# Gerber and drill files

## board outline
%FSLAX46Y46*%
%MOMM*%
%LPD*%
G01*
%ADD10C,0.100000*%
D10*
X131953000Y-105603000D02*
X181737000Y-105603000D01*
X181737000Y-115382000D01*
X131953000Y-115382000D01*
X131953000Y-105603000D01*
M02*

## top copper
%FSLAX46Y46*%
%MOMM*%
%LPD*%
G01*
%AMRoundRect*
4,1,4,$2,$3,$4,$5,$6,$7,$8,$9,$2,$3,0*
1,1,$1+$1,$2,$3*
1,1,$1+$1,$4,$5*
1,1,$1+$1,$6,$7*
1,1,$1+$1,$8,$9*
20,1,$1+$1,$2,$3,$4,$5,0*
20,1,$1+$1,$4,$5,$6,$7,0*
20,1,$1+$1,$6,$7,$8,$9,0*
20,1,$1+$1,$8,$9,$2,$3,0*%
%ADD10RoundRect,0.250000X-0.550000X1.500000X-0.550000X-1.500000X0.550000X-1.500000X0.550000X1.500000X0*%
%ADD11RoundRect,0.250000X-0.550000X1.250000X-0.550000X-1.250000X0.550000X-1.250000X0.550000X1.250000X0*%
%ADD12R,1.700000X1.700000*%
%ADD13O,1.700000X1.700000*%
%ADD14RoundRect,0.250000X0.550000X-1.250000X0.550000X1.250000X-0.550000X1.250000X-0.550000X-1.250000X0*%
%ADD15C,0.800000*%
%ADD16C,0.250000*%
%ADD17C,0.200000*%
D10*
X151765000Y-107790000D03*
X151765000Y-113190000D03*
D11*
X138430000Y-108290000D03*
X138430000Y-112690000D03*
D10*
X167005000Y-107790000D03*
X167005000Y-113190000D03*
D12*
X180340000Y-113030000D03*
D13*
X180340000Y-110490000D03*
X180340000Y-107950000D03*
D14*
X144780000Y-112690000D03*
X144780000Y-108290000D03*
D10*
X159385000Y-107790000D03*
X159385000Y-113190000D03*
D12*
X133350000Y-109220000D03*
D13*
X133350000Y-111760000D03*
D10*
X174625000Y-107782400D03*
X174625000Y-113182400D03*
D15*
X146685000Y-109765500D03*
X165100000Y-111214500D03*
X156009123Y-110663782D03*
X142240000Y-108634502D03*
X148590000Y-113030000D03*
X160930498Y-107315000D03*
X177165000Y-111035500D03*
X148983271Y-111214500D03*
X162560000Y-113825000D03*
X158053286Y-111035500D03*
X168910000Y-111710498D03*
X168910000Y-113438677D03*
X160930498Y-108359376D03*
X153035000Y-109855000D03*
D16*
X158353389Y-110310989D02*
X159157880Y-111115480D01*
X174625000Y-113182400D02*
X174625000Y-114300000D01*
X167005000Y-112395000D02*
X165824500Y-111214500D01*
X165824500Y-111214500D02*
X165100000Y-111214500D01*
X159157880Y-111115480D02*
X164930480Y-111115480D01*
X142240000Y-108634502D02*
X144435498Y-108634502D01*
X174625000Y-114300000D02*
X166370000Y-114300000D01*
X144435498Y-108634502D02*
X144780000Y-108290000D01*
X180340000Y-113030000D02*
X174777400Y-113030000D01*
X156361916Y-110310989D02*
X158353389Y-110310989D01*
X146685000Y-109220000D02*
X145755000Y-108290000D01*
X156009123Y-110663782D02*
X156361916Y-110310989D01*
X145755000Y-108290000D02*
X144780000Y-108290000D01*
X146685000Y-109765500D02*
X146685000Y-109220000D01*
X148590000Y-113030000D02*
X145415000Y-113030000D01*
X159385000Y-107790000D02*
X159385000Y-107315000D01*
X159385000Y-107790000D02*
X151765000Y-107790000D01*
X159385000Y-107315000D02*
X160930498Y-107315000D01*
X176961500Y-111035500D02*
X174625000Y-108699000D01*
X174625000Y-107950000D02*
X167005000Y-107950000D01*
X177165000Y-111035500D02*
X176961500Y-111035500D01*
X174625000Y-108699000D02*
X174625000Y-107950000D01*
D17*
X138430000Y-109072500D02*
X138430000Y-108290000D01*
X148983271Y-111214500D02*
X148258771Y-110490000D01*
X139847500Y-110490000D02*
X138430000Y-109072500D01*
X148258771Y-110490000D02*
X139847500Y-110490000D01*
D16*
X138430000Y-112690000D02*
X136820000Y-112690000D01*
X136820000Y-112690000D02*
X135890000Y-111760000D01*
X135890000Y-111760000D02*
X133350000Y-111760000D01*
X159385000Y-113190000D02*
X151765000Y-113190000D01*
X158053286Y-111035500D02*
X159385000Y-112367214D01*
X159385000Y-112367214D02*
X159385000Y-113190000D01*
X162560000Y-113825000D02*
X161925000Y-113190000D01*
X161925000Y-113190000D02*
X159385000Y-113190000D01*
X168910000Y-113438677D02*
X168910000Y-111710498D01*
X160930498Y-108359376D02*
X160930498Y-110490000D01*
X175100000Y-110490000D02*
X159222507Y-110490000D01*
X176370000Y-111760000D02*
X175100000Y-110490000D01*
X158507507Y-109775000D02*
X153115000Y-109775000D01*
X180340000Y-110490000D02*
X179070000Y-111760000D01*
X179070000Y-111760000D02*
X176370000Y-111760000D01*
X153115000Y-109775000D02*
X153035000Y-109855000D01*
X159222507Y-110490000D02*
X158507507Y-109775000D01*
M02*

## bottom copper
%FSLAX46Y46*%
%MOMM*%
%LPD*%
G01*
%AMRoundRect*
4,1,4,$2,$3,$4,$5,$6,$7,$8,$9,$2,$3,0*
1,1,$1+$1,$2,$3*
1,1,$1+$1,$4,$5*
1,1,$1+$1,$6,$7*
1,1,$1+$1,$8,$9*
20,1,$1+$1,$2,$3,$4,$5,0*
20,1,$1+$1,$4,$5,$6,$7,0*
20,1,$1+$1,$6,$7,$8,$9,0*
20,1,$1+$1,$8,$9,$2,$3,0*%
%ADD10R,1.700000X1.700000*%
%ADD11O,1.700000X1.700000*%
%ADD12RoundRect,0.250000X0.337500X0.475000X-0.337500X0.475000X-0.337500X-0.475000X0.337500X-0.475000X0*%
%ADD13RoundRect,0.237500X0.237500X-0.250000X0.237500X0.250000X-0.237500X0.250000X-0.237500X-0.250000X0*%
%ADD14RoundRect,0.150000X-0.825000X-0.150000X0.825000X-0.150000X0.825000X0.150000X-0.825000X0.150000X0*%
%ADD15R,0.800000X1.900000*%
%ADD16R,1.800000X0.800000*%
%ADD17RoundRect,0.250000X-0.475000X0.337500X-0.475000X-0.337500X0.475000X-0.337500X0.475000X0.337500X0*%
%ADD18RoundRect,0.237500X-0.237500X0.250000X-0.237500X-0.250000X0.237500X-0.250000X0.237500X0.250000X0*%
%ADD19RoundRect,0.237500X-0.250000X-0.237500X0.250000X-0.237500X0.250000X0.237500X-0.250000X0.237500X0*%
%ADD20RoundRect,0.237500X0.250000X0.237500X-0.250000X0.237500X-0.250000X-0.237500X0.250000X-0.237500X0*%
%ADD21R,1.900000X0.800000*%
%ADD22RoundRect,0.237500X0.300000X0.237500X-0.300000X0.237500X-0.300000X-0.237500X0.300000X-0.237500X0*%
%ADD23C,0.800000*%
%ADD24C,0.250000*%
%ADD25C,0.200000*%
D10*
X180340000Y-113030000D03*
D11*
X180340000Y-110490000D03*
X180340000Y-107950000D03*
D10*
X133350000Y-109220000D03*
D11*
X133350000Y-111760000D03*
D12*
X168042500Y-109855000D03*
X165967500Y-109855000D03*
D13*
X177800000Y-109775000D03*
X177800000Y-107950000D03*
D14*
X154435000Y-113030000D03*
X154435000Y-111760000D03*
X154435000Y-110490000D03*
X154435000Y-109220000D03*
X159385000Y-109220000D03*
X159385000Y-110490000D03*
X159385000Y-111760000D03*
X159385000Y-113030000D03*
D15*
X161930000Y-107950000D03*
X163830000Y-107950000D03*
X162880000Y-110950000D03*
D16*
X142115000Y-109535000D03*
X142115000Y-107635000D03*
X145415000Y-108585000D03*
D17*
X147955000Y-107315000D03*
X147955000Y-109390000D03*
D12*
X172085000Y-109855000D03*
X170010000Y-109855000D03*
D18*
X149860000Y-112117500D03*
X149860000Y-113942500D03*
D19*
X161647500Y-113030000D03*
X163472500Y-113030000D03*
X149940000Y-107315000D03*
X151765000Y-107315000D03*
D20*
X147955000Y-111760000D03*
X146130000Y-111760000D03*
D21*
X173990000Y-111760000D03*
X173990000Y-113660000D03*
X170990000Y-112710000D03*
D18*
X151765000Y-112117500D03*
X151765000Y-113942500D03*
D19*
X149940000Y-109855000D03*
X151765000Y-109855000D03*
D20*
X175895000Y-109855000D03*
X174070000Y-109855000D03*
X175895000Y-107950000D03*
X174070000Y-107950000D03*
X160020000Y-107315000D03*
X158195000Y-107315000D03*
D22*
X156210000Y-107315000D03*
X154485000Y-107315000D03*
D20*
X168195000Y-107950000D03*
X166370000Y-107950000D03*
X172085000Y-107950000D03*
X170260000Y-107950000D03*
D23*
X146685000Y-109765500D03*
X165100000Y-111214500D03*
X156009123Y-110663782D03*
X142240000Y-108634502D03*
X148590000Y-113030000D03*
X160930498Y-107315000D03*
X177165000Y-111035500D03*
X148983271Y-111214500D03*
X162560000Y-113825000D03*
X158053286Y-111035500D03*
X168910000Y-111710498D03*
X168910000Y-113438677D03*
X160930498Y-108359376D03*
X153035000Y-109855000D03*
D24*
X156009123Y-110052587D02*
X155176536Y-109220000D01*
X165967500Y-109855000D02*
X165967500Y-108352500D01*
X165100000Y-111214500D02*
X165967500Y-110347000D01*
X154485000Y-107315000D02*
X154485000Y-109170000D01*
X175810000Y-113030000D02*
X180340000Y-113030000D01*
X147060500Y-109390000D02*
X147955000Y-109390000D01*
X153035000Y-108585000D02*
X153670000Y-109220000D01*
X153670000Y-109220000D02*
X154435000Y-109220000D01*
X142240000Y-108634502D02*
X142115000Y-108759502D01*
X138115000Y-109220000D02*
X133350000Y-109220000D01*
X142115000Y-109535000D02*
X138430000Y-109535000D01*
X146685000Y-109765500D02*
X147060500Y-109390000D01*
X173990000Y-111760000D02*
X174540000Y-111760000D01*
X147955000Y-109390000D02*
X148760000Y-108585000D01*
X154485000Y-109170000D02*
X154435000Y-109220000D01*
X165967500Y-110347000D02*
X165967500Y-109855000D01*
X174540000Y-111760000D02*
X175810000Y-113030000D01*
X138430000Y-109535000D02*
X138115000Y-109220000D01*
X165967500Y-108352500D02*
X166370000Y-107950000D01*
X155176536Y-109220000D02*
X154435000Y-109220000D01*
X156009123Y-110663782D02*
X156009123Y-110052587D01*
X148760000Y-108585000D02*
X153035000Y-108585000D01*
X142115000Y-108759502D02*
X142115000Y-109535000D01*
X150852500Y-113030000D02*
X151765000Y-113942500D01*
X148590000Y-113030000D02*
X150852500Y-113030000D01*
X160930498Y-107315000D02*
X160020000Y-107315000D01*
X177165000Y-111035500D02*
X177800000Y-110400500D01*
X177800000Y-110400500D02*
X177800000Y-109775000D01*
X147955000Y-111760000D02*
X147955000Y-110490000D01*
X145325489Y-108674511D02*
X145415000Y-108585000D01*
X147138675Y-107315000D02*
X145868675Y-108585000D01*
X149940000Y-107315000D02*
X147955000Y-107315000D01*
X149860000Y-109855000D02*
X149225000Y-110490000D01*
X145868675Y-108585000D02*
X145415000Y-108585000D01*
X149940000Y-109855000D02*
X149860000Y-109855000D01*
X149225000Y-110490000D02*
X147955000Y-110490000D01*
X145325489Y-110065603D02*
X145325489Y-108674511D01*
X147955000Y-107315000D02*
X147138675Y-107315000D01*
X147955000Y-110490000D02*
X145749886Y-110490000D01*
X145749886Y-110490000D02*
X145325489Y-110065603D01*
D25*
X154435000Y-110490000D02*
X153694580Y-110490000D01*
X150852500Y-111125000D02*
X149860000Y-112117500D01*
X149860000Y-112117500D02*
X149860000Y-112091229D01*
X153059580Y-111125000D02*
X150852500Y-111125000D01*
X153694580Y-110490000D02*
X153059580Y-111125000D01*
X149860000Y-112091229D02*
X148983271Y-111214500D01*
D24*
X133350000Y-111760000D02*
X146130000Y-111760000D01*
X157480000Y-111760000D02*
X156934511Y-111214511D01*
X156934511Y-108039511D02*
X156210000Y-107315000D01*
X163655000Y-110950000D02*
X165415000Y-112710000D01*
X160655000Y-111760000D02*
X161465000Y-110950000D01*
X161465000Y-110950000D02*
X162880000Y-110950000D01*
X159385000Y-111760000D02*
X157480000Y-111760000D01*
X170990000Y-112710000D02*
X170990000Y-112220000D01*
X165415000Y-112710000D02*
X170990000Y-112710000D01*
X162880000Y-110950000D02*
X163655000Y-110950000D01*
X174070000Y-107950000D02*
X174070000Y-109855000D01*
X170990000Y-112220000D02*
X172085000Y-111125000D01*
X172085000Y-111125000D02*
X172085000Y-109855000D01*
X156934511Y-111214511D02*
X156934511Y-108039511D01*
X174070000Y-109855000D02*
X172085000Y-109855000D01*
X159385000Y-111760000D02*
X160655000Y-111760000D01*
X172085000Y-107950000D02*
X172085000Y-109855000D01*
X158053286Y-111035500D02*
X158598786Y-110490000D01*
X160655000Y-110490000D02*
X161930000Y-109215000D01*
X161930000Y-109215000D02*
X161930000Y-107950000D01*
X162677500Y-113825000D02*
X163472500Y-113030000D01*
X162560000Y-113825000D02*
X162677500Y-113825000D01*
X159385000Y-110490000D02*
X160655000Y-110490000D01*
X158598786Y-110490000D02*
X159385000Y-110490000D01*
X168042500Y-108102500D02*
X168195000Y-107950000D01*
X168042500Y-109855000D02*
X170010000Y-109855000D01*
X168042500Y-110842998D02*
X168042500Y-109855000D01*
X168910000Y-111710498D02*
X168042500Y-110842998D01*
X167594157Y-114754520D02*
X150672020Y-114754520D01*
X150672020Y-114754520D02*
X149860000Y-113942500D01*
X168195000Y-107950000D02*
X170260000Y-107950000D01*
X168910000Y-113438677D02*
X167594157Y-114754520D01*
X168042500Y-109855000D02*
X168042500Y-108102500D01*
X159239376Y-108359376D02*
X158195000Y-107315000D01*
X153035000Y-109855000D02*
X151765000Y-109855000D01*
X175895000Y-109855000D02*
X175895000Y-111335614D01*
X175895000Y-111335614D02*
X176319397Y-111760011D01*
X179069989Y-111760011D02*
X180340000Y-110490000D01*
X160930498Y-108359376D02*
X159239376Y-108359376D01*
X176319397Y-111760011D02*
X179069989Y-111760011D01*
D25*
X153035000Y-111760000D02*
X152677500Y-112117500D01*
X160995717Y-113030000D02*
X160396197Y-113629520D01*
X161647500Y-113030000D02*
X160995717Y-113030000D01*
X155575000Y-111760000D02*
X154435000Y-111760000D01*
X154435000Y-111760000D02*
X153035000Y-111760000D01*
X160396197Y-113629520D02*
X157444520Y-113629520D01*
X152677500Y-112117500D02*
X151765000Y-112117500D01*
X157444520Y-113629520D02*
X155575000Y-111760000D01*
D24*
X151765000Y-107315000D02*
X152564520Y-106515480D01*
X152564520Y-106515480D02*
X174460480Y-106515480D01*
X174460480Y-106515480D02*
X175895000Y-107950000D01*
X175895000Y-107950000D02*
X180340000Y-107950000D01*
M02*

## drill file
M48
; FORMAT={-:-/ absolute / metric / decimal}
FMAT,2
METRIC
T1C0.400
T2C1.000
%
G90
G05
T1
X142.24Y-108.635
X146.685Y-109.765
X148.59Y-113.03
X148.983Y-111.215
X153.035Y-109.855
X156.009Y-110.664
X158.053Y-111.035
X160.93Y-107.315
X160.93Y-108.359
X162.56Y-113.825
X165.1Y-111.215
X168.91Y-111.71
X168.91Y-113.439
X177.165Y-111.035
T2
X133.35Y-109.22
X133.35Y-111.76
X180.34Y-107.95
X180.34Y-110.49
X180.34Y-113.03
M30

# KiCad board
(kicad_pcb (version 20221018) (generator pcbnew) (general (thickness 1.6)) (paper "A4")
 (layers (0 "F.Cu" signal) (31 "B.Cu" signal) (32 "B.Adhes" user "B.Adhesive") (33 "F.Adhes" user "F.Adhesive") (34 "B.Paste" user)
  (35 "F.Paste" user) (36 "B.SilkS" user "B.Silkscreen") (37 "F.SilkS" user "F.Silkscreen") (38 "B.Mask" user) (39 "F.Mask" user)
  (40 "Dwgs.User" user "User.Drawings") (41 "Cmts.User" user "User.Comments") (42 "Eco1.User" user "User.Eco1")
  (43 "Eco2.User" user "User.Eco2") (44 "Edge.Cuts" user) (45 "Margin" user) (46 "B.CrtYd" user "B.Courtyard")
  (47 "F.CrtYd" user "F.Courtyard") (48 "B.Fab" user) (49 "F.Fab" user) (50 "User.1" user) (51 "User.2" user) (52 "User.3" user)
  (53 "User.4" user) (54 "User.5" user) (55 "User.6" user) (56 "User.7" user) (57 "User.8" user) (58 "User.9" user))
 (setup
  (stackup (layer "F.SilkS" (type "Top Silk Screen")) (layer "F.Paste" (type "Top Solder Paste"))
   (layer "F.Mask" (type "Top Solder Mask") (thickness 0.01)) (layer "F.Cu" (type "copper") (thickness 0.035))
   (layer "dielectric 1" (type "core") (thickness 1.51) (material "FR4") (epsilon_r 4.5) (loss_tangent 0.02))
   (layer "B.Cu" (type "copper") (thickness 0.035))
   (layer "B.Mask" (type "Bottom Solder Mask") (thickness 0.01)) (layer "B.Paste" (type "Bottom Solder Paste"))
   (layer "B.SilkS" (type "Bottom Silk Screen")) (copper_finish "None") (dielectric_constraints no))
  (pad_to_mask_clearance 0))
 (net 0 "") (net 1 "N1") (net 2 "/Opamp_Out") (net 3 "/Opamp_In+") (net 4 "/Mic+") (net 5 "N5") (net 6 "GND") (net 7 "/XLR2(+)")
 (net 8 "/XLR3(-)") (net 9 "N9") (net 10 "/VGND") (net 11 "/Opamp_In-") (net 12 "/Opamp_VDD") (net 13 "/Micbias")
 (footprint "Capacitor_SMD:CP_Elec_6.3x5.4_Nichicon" (layer "F.Cu") (at 151.765 110.49 -90)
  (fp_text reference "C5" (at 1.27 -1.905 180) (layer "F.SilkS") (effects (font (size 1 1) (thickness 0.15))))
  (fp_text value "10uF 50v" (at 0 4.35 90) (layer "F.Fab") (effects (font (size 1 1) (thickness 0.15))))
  (pad "1" smd roundrect (at -2.7 0 270) (size 3.5 1.6) (layers "F.Cu" "F.Paste" "F.Mask") (roundrect_rratio 0.15625) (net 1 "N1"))
  (pad "2" smd roundrect (at 2.7 0 270) (size 3.5 1.6) (layers "F.Cu" "F.Paste" "F.Mask") (roundrect_rratio 0.15625) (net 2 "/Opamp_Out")))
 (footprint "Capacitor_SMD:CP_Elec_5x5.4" (layer "F.Cu") (at 138.43 110.49 -90)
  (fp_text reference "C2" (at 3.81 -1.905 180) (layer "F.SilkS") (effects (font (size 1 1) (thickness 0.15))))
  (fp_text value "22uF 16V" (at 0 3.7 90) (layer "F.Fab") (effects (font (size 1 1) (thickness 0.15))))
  (pad "1" smd roundrect (at -2.2 0 270) (size 3 1.6) (layers "F.Cu" "F.Paste" "F.Mask") (roundrect_rratio 0.15625) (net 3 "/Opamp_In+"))
  (pad "2" smd roundrect (at 2.2 0 270) (size 3 1.6) (layers "F.Cu" "F.Paste" "F.Mask") (roundrect_rratio 0.15625) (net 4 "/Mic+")))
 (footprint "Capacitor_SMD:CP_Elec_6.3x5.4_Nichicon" (layer "F.Cu") (at 167.005 110.49 -90)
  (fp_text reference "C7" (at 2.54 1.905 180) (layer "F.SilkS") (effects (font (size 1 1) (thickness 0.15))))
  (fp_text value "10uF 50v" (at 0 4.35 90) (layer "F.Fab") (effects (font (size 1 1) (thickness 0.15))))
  (pad "1" smd roundrect (at -2.7 0 270) (size 3.5 1.6) (layers "F.Cu" "F.Paste" "F.Mask") (roundrect_rratio 0.15625) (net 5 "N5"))
  (pad "2" smd roundrect (at 2.7 0 270) (size 3.5 1.6) (layers "F.Cu" "F.Paste" "F.Mask") (roundrect_rratio 0.15625) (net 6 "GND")))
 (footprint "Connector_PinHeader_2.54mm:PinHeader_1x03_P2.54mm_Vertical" (layer "F.Cu") (at 180.34 113.03 180)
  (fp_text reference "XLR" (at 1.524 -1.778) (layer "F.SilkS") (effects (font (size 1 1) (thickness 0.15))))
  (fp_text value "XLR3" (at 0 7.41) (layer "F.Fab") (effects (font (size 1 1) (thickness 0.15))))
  (pad "1" thru_hole rect (at 0 0 180) (size 1.7 1.7) (drill 1) (layers "*.Cu" "*.Mask") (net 6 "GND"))
  (pad "2" thru_hole oval (at 0 2.54 180) (size 1.7 1.7) (drill 1) (layers "*.Cu" "*.Mask") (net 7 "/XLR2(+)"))
  (pad "3" thru_hole oval (at 0 5.08 180) (size 1.7 1.7) (drill 1) (layers "*.Cu" "*.Mask") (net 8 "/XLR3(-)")))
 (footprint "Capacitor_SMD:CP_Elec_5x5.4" (layer "F.Cu") (at 144.78 110.49 90)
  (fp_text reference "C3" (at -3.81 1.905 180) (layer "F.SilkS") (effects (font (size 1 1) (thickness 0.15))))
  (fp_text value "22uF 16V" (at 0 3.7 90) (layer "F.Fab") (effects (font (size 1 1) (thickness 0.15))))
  (pad "1" smd roundrect (at -2.2 0 90) (size 3 1.6) (layers "F.Cu" "F.Paste" "F.Mask") (roundrect_rratio 0.15625) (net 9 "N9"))
  (pad "2" smd roundrect (at 2.2 0 90) (size 3 1.6) (layers "F.Cu" "F.Paste" "F.Mask") (roundrect_rratio 0.15625) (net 6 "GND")))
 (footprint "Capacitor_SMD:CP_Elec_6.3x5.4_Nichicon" (layer "F.Cu") (at 159.385 110.49 -90)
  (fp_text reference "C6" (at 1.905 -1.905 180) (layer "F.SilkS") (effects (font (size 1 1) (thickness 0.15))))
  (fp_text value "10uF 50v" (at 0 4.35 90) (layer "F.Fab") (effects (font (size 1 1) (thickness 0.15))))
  (pad "1" smd roundrect (at -2.7 0 270) (size 3.5 1.6) (layers "F.Cu" "F.Paste" "F.Mask") (roundrect_rratio 0.15625) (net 1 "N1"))
  (pad "2" smd roundrect (at 2.7 0 270) (size 3.5 1.6) (layers "F.Cu" "F.Paste" "F.Mask") (roundrect_rratio 0.15625) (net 2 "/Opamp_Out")))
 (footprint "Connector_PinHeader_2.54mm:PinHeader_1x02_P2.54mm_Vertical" (layer "F.Cu") (at 133.35 109.22)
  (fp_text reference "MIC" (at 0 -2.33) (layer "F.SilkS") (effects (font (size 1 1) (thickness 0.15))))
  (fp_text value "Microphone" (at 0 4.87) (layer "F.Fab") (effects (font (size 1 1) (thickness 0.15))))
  (pad "1" thru_hole rect (at 0 0) (size 1.7 1.7) (drill 1) (layers "*.Cu" "*.Mask") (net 6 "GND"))
  (pad "2" thru_hole oval (at 0 2.54) (size 1.7 1.7) (drill 1) (layers "*.Cu" "*.Mask") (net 4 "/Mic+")))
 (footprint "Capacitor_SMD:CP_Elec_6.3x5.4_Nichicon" (layer "F.Cu") (at 174.625 110.4824 -90)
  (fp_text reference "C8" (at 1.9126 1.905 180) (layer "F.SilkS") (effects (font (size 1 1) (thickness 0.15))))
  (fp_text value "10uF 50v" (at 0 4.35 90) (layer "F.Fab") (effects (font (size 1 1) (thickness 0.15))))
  (pad "1" smd roundrect (at -2.7 0 270) (size 3.5 1.6) (layers "F.Cu" "F.Paste" "F.Mask") (roundrect_rratio 0.15625) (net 5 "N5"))
  (pad "2" smd roundrect (at 2.7 0 270) (size 3.5 1.6) (layers "F.Cu" "F.Paste" "F.Mask") (roundrect_rratio 0.15625) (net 6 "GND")))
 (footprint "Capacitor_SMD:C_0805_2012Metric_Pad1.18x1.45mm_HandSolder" (layer "B.Cu") (at 167.005 109.855 180)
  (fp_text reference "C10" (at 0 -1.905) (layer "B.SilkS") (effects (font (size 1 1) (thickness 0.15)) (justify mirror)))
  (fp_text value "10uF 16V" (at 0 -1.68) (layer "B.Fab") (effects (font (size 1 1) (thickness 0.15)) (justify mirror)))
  (pad "1" smd roundrect (at -1.0375 0 180) (size 1.175 1.45) (layers "B.Cu" "B.Paste" "B.Mask") (roundrect_rratio 0.2127659574)
   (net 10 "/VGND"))
  (pad "2" smd roundrect (at 1.0375 0 180) (size 1.175 1.45) (layers "B.Cu" "B.Paste" "B.Mask") (roundrect_rratio 0.2127659574)
   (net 6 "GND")))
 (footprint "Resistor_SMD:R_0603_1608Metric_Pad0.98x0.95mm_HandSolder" (layer "B.Cu") (at 177.8 108.8625 90)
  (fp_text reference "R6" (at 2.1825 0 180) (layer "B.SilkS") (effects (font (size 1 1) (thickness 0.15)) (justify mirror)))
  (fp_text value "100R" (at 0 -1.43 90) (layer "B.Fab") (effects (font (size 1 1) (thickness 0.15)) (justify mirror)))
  (pad "1" smd roundrect (at -0.9125 0 90) (size 0.975 0.95) (layers "B.Cu" "B.Paste" "B.Mask") (roundrect_rratio 0.25) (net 5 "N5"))
  (pad "2" smd roundrect (at 0.9125 0 90) (size 0.975 0.95) (layers "B.Cu" "B.Paste" "B.Mask") (roundrect_rratio 0.25) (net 8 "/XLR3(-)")))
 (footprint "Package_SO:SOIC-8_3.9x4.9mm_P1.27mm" (layer "B.Cu") (at 156.91 111.125)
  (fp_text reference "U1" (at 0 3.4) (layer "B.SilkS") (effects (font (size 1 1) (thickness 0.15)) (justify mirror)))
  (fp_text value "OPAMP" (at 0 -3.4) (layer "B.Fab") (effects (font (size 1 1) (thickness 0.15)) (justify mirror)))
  (pad "1" smd roundrect (at -2.475 1.905) (size 1.95 0.6) (layers "B.Cu" "B.Paste" "B.Mask") (roundrect_rratio 0.25))
  (pad "2" smd roundrect (at -2.475 0.635) (size 1.95 0.6) (layers "B.Cu" "B.Paste" "B.Mask") (roundrect_rratio 0.25) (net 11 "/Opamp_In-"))
  (pad "3" smd roundrect (at -2.475 -0.635) (size 1.95 0.6) (layers "B.Cu" "B.Paste" "B.Mask") (roundrect_rratio 0.25) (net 3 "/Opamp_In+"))
  (pad "4" smd roundrect (at -2.475 -1.905) (size 1.95 0.6) (layers "B.Cu" "B.Paste" "B.Mask") (roundrect_rratio 0.25) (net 6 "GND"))
  (pad "5" smd roundrect (at 2.475 -1.905) (size 1.95 0.6) (layers "B.Cu" "B.Paste" "B.Mask") (roundrect_rratio 0.25))
  (pad "6" smd roundrect (at 2.475 -0.635) (size 1.95 0.6) (layers "B.Cu" "B.Paste" "B.Mask") (roundrect_rratio 0.25) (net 2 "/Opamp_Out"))
  (pad "7" smd roundrect (at 2.475 0.635) (size 1.95 0.6) (layers "B.Cu" "B.Paste" "B.Mask") (roundrect_rratio 0.25) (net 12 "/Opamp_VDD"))
  (pad "8" smd roundrect (at 2.475 1.905) (size 1.95 0.6) (layers "B.Cu" "B.Paste" "B.Mask") (roundrect_rratio 0.25)))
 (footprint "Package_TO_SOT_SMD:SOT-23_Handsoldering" (layer "B.Cu") (at 162.88 109.45 -90)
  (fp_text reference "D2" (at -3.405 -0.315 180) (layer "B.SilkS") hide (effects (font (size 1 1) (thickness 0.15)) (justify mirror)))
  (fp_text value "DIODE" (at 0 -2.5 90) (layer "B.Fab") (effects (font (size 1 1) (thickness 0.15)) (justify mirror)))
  (pad "1" smd rect (at -1.5 0.95 270) (size 1.9 0.8) (layers "B.Cu" "B.Paste" "B.Mask") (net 2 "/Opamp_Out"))
  (pad "2" smd rect (at -1.5 -0.95 270) (size 1.9 0.8) (layers "B.Cu" "B.Paste" "B.Mask"))
  (pad "3" smd rect (at 1.5 0 270) (size 1.9 0.8) (layers "B.Cu" "B.Paste" "B.Mask") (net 12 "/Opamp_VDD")))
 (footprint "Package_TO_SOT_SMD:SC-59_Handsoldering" (layer "B.Cu") (at 143.765 108.585)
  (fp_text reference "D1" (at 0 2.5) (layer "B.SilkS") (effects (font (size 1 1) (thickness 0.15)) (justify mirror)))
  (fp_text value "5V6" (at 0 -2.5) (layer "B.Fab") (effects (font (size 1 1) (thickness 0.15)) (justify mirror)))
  (pad "1" smd rect (at -1.65 0.95) (size 1.8 0.8) (layers "B.Cu" "B.Paste" "B.Mask") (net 6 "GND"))
  (pad "2" smd rect (at -1.65 -0.95) (size 1.8 0.8) (layers "B.Cu" "B.Paste" "B.Mask"))
  (pad "3" smd rect (at 1.65 0) (size 1.8 0.8) (layers "B.Cu" "B.Paste" "B.Mask") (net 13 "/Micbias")))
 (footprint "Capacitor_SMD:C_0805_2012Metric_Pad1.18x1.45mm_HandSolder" (layer "B.Cu") (at 147.955 108.3525 -90)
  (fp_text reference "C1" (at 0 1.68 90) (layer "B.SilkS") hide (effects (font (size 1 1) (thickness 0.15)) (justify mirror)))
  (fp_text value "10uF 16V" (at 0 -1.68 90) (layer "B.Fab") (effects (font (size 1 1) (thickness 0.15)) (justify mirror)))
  (pad "1" smd roundrect (at -1.0375 0 270) (size 1.175 1.45) (layers "B.Cu" "B.Paste" "B.Mask") (roundrect_rratio 0.2127659574)
   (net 13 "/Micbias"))
  (pad "2" smd roundrect (at 1.0375 0 270) (size 1.175 1.45) (layers "B.Cu" "B.Paste" "B.Mask") (roundrect_rratio 0.2127659574)
   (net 6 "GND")))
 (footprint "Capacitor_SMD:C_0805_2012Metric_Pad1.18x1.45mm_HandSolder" (layer "B.Cu") (at 171.0475 109.855 180)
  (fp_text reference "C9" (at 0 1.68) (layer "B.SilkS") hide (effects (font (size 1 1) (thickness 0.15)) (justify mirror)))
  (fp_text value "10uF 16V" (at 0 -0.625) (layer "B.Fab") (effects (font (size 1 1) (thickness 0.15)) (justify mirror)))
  (pad "1" smd roundrect (at -1.0375 0 180) (size 1.175 1.45) (layers "B.Cu" "B.Paste" "B.Mask") (roundrect_rratio 0.2127659574)
   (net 12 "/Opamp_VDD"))
  (pad "2" smd roundrect (at 1.0375 0 180) (size 1.175 1.45) (layers "B.Cu" "B.Paste" "B.Mask") (roundrect_rratio 0.2127659574)
   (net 10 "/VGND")))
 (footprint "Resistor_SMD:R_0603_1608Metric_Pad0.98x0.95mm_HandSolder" (layer "B.Cu") (at 149.86 113.03 -90)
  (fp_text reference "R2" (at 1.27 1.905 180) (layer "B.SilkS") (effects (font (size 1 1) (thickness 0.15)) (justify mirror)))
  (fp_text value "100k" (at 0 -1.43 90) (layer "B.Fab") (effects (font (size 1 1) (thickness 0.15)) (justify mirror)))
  (pad "1" smd roundrect (at -0.9125 0 270) (size 0.975 0.95) (layers "B.Cu" "B.Paste" "B.Mask") (roundrect_rratio 0.25)
   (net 3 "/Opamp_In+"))
  (pad "2" smd roundrect (at 0.9125 0 270) (size 0.975 0.95) (layers "B.Cu" "B.Paste" "B.Mask") (roundrect_rratio 0.25) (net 10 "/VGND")))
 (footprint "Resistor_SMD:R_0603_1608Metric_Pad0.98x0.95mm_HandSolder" (layer "B.Cu") (at 162.56 113.03)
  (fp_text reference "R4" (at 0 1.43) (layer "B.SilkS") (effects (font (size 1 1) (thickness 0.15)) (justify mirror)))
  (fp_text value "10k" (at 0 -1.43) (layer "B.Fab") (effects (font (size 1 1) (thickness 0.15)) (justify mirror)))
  (pad "1" smd roundrect (at -0.9125 0) (size 0.975 0.95) (layers "B.Cu" "B.Paste" "B.Mask") (roundrect_rratio 0.25) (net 11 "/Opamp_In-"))
  (pad "2" smd roundrect (at 0.9125 0) (size 0.975 0.95) (layers "B.Cu" "B.Paste" "B.Mask") (roundrect_rratio 0.25) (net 2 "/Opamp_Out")))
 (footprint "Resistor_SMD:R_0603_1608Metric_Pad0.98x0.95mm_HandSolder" (layer "B.Cu") (at 150.8525 107.315)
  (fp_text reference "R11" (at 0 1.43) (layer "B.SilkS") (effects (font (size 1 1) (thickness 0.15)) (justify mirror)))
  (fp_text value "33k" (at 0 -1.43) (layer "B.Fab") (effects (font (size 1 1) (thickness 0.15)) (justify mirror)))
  (pad "1" smd roundrect (at -0.9125 0) (size 0.975 0.95) (layers "B.Cu" "B.Paste" "B.Mask") (roundrect_rratio 0.25) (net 13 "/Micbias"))
  (pad "2" smd roundrect (at 0.9125 0) (size 0.975 0.95) (layers "B.Cu" "B.Paste" "B.Mask") (roundrect_rratio 0.25) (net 8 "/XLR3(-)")))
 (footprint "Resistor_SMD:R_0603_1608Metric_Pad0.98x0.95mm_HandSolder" (layer "B.Cu") (at 147.0425 111.76 180)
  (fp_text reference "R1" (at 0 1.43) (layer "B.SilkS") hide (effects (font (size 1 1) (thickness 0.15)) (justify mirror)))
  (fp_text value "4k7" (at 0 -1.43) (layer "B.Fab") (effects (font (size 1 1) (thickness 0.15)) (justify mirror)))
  (pad "1" smd roundrect (at -0.9125 0 180) (size 0.975 0.95) (layers "B.Cu" "B.Paste" "B.Mask") (roundrect_rratio 0.25) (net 13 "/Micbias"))
  (pad "2" smd roundrect (at 0.9125 0 180) (size 0.975 0.95) (layers "B.Cu" "B.Paste" "B.Mask") (roundrect_rratio 0.25) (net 4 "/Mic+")))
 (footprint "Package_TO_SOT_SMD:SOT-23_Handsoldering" (layer "B.Cu") (at 172.49 112.71 180)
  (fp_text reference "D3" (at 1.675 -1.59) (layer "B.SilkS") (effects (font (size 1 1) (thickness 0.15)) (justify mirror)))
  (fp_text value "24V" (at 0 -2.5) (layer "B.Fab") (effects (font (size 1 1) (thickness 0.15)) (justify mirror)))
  (pad "1" smd rect (at -1.5 0.95 180) (size 1.9 0.8) (layers "B.Cu" "B.Paste" "B.Mask") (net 6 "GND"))
  (pad "2" smd rect (at -1.5 -0.95 180) (size 1.9 0.8) (layers "B.Cu" "B.Paste" "B.Mask"))
  (pad "3" smd rect (at 1.5 0 180) (size 1.9 0.8) (layers "B.Cu" "B.Paste" "B.Mask") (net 12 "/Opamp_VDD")))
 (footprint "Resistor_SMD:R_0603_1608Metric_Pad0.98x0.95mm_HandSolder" (layer "B.Cu") (at 151.765 113.03 -90)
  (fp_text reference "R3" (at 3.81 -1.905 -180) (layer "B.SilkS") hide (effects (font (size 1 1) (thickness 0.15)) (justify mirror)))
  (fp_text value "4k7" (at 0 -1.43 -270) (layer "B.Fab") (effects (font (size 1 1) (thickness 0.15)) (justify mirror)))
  (pad "1" smd roundrect (at -0.9125 0 270) (size 0.975 0.95) (layers "B.Cu" "B.Paste" "B.Mask") (roundrect_rratio 0.25)
   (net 11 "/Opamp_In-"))
  (pad "2" smd roundrect (at 0.9125 0 270) (size 0.975 0.95) (layers "B.Cu" "B.Paste" "B.Mask") (roundrect_rratio 0.25) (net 9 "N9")))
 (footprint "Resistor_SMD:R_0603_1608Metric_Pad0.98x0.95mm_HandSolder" (layer "B.Cu") (at 150.8525 109.855)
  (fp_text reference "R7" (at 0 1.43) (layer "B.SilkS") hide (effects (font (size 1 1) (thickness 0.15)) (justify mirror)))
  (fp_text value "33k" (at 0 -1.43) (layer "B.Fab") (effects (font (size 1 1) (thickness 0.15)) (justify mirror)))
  (pad "1" smd roundrect (at -0.9125 0) (size 0.975 0.95) (layers "B.Cu" "B.Paste" "B.Mask") (roundrect_rratio 0.25) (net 13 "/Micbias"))
  (pad "2" smd roundrect (at 0.9125 0) (size 0.975 0.95) (layers "B.Cu" "B.Paste" "B.Mask") (roundrect_rratio 0.25) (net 7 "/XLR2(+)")))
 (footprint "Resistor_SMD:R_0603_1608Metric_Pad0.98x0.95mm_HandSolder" (layer "B.Cu") (at 174.9825 109.855 180)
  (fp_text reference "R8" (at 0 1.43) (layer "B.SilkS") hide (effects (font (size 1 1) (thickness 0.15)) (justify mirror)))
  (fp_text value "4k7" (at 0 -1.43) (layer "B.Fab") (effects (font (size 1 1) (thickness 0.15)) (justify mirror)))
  (pad "1" smd roundrect (at -0.9125 0 180) (size 0.975 0.95) (layers "B.Cu" "B.Paste" "B.Mask") (roundrect_rratio 0.25) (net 7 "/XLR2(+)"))
  (pad "2" smd roundrect (at 0.9125 0 180) (size 0.975 0.95) (layers "B.Cu" "B.Paste" "B.Mask") (roundrect_rratio 0.25)
   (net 12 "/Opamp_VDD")))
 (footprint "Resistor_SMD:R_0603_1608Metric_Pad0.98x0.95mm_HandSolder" (layer "B.Cu") (at 174.9825 107.95 180)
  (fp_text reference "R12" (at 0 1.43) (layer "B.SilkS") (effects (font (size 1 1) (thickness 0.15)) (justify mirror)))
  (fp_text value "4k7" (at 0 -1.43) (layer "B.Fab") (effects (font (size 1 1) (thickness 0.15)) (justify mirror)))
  (pad "1" smd roundrect (at -0.9125 0 180) (size 0.975 0.95) (layers "B.Cu" "B.Paste" "B.Mask") (roundrect_rratio 0.25) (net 8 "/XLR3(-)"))
  (pad "2" smd roundrect (at 0.9125 0 180) (size 0.975 0.95) (layers "B.Cu" "B.Paste" "B.Mask") (roundrect_rratio 0.25)
   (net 12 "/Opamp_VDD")))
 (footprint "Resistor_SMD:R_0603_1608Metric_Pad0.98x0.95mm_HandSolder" (layer "B.Cu") (at 159.1075 107.315 180)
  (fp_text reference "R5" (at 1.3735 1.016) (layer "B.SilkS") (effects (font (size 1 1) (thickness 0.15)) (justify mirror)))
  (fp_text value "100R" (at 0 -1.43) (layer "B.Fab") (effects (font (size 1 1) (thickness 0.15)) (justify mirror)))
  (pad "1" smd roundrect (at -0.9125 0 180) (size 0.975 0.95) (layers "B.Cu" "B.Paste" "B.Mask") (roundrect_rratio 0.25) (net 1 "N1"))
  (pad "2" smd roundrect (at 0.9125 0 180) (size 0.975 0.95) (layers "B.Cu" "B.Paste" "B.Mask") (roundrect_rratio 0.25) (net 7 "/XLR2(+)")))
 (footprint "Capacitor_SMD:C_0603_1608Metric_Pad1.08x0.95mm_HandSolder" (layer "B.Cu") (at 155.3475 107.315 180)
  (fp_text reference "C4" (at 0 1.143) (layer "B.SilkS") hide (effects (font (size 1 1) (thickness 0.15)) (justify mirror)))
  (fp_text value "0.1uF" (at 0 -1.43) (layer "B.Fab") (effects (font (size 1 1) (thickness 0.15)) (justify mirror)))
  (pad "1" smd roundrect (at -0.8625 0 180) (size 1.075 0.95) (layers "B.Cu" "B.Paste" "B.Mask") (roundrect_rratio 0.25)
   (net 12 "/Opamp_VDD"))
  (pad "2" smd roundrect (at 0.8625 0 180) (size 1.075 0.95) (layers "B.Cu" "B.Paste" "B.Mask") (roundrect_rratio 0.25) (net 6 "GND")))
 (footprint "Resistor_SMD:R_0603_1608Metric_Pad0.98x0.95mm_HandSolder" (layer "B.Cu") (at 167.2825 107.95 180)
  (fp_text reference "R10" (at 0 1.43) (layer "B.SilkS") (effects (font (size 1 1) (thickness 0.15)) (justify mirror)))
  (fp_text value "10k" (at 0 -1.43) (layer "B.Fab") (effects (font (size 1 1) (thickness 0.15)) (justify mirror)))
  (pad "1" smd roundrect (at -0.9125 0 180) (size 0.975 0.95) (layers "B.Cu" "B.Paste" "B.Mask") (roundrect_rratio 0.25) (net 10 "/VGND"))
  (pad "2" smd roundrect (at 0.9125 0 180) (size 0.975 0.95) (layers "B.Cu" "B.Paste" "B.Mask") (roundrect_rratio 0.25) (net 6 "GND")))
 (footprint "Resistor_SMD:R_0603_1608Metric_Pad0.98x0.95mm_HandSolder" (layer "B.Cu") (at 171.1725 107.95 180)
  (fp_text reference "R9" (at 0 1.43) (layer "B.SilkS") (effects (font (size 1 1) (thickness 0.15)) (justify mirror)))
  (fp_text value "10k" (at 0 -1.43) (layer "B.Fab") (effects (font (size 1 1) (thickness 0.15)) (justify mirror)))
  (pad "1" smd roundrect (at -0.9125 0 180) (size 0.975 0.95) (layers "B.Cu" "B.Paste" "B.Mask") (roundrect_rratio 0.25)
   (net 12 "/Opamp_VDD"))
  (pad "2" smd roundrect (at 0.9125 0 180) (size 0.975 0.95) (layers "B.Cu" "B.Paste" "B.Mask") (roundrect_rratio 0.25) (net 10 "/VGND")))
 (gr_rect (start 131.953 105.603) (end 181.737 115.382) (stroke (width 0.1) (type solid)) (fill none) (layer "Edge.Cuts"))
 (segment (start 158.353389 110.310989) (end 159.15788 111.11548) (width 0.25) (layer "F.Cu") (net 6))
 (segment (start 174.625 113.1824) (end 174.625 114.3) (width 0.25) (layer "F.Cu") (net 6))
 (segment (start 167.005 112.395) (end 165.8245 111.2145) (width 0.25) (layer "F.Cu") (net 6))
 (segment (start 165.8245 111.2145) (end 165.1 111.2145) (width 0.25) (layer "F.Cu") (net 6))
 (segment (start 159.15788 111.11548) (end 164.93048 111.11548) (width 0.25) (layer "F.Cu") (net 6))
 (segment (start 142.24 108.634502) (end 144.435498 108.634502) (width 0.25) (layer "F.Cu") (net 6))
 (segment (start 174.625 114.3) (end 166.37 114.3) (width 0.25) (layer "F.Cu") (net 6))
 (segment (start 144.435498 108.634502) (end 144.78 108.29) (width 0.25) (layer "F.Cu") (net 6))
 (segment (start 180.34 113.03) (end 174.7774 113.03) (width 0.25) (layer "F.Cu") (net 6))
 (segment (start 156.361916 110.310989) (end 158.353389 110.310989) (width 0.25) (layer "F.Cu") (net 6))
 (segment (start 146.685 109.22) (end 145.755 108.29) (width 0.25) (layer "F.Cu") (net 6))
 (segment (start 156.009123 110.663782) (end 156.361916 110.310989) (width 0.25) (layer "F.Cu") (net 6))
 (segment (start 145.755 108.29) (end 144.78 108.29) (width 0.25) (layer "F.Cu") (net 6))
 (segment (start 146.685 109.7655) (end 146.685 109.22) (width 0.25) (layer "F.Cu") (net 6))
 (via (at 146.685 109.7655) (size 0.8) (drill 0.4) (layers "F.Cu" "B.Cu") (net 6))
 (via (at 165.1 111.2145) (size 0.8) (drill 0.4) (layers "F.Cu" "B.Cu") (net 6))
 (via (at 156.009123 110.663782) (size 0.8) (drill 0.4) (layers "F.Cu" "B.Cu") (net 6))
 (via (at 142.24 108.634502) (size 0.8) (drill 0.4) (layers "F.Cu" "B.Cu") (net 6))
 (segment (start 156.009123 110.052587) (end 155.176536 109.22) (width 0.25) (layer "B.Cu") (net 6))
 (segment (start 165.9675 109.855) (end 165.9675 108.3525) (width 0.25) (layer "B.Cu") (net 6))
 (segment (start 165.1 111.2145) (end 165.9675 110.347) (width 0.25) (layer "B.Cu") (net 6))
 (segment (start 154.485 107.315) (end 154.485 109.17) (width 0.25) (layer "B.Cu") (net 6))
 (segment (start 175.81 113.03) (end 180.34 113.03) (width 0.25) (layer "B.Cu") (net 6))
 (segment (start 147.0605 109.39) (end 147.955 109.39) (width 0.25) (layer "B.Cu") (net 6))
 (segment (start 153.035 108.585) (end 153.67 109.22) (width 0.25) (layer "B.Cu") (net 6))
 (segment (start 153.67 109.22) (end 154.435 109.22) (width 0.25) (layer "B.Cu") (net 6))
 (segment (start 142.24 108.634502) (end 142.115 108.759502) (width 0.25) (layer "B.Cu") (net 6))
 (segment (start 138.115 109.22) (end 133.35 109.22) (width 0.25) (layer "B.Cu") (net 6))
 (segment (start 142.115 109.535) (end 138.43 109.535) (width 0.25) (layer "B.Cu") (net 6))
 (segment (start 146.685 109.7655) (end 147.0605 109.39) (width 0.25) (layer "B.Cu") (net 6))
 (segment (start 173.99 111.76) (end 174.54 111.76) (width 0.25) (layer "B.Cu") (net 6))
 (segment (start 147.955 109.39) (end 148.76 108.585) (width 0.25) (layer "B.Cu") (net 6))
 (segment (start 154.485 109.17) (end 154.435 109.22) (width 0.25) (layer "B.Cu") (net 6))
 (segment (start 165.9675 110.347) (end 165.9675 109.855) (width 0.25) (layer "B.Cu") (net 6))
 (segment (start 174.54 111.76) (end 175.81 113.03) (width 0.25) (layer "B.Cu") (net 6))
 (segment (start 138.43 109.535) (end 138.115 109.22) (width 0.25) (layer "B.Cu") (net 6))
 (segment (start 165.9675 108.3525) (end 166.37 107.95) (width 0.25) (layer "B.Cu") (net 6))
 (segment (start 155.176536 109.22) (end 154.435 109.22) (width 0.25) (layer "B.Cu") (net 6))
 (segment (start 156.009123 110.663782) (end 156.009123 110.052587) (width 0.25) (layer "B.Cu") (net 6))
 (segment (start 148.76 108.585) (end 153.035 108.585) (width 0.25) (layer "B.Cu") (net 6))
 (segment (start 142.115 108.759502) (end 142.115 109.535) (width 0.25) (layer "B.Cu") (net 6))
 (segment (start 148.59 113.03) (end 145.415 113.03) (width 0.25) (layer "F.Cu") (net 9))
 (via (at 148.59 113.03) (size 0.8) (drill 0.4) (layers "F.Cu" "B.Cu") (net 9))
 (segment (start 150.8525 113.03) (end 151.765 113.9425) (width 0.25) (layer "B.Cu") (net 9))
 (segment (start 148.59 113.03) (end 150.8525 113.03) (width 0.25) (layer "B.Cu") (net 9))
 (segment (start 159.385 107.79) (end 159.385 107.315) (width 0.25) (layer "F.Cu") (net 1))
 (segment (start 159.385 107.79) (end 151.765 107.79) (width 0.25) (layer "F.Cu") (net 1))
 (segment (start 159.385 107.315) (end 160.930498 107.315) (width 0.25) (layer "F.Cu") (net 1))
 (via (at 160.930498 107.315) (size 0.8) (drill 0.4) (layers "F.Cu" "B.Cu") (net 1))
 (segment (start 160.930498 107.315) (end 160.02 107.315) (width 0.25) (layer "B.Cu") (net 1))
 (segment (start 176.9615 111.0355) (end 174.625 108.699) (width 0.25) (layer "F.Cu") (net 5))
 (segment (start 174.625 107.95) (end 167.005 107.95) (width 0.25) (layer "F.Cu") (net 5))
 (segment (start 177.165 111.0355) (end 176.9615 111.0355) (width 0.25) (layer "F.Cu") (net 5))
 (segment (start 174.625 108.699) (end 174.625 107.95) (width 0.25) (layer "F.Cu") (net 5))
 (via (at 177.165 111.0355) (size 0.8) (drill 0.4) (layers "F.Cu" "B.Cu") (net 5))
 (segment (start 177.165 111.0355) (end 177.8 110.4005) (width 0.25) (layer "B.Cu") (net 5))
 (segment (start 177.8 110.4005) (end 177.8 109.775) (width 0.25) (layer "B.Cu") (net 5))
 (segment (start 147.955 111.76) (end 147.955 110.49) (width 0.25) (layer "B.Cu") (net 13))
 (segment (start 145.325489 108.674511) (end 145.415 108.585) (width 0.25) (layer "B.Cu") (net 13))
 (segment (start 147.138675 107.315) (end 145.868675 108.585) (width 0.25) (layer "B.Cu") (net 13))
 (segment (start 149.94 107.315) (end 147.955 107.315) (width 0.25) (layer "B.Cu") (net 13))
 (segment (start 149.86 109.855) (end 149.225 110.49) (width 0.25) (layer "B.Cu") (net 13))
 (segment (start 145.868675 108.585) (end 145.415 108.585) (width 0.25) (layer "B.Cu") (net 13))
 (segment (start 149.94 109.855) (end 149.86 109.855) (width 0.25) (layer "B.Cu") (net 13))
 (segment (start 149.225 110.49) (end 147.955 110.49) (width 0.25) (layer "B.Cu") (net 13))
 (segment (start 145.325489 110.065603) (end 145.325489 108.674511) (width 0.25) (layer "B.Cu") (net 13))
 (segment (start 147.955 107.315) (end 147.138675 107.315) (width 0.25) (layer "B.Cu") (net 13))
 (segment (start 147.955 110.49) (end 145.749886 110.49) (width 0.25) (layer "B.Cu") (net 13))
 (segment (start 145.749886 110.49) (end 145.325489 110.065603) (width 0.25) (layer "B.Cu") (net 13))
 (segment (start 138.43 109.0725) (end 138.43 108.29) (width 0.2) (layer "F.Cu") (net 3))
 (segment (start 148.983271 111.2145) (end 148.258771 110.49) (width 0.2) (layer "F.Cu") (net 3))
 (segment (start 139.8475 110.49) (end 138.43 109.0725) (width 0.2) (layer "F.Cu") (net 3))
 (segment (start 148.258771 110.49) (end 139.8475 110.49) (width 0.2) (layer "F.Cu") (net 3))
 (via (at 148.983271 111.2145) (size 0.8) (drill 0.4) (layers "F.Cu" "B.Cu") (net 3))
 (segment (start 154.435 110.49) (end 153.69458 110.49) (width 0.2) (layer "B.Cu") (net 3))
 (segment (start 150.8525 111.125) (end 149.86 112.1175) (width 0.2) (layer "B.Cu") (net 3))
 (segment (start 149.86 112.1175) (end 149.86 112.091229) (width 0.2) (layer "B.Cu") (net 3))
 (segment (start 153.05958 111.125) (end 150.8525 111.125) (width 0.2) (layer "B.Cu") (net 3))
 (segment (start 153.69458 110.49) (end 153.05958 111.125) (width 0.2) (layer "B.Cu") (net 3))
 (segment (start 149.86 112.091229) (end 148.983271 111.2145) (width 0.2) (layer "B.Cu") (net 3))
 (segment (start 138.43 112.69) (end 136.82 112.69) (width 0.25) (layer "F.Cu") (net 4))
 (segment (start 136.82 112.69) (end 135.89 111.76) (width 0.25) (layer "F.Cu") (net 4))
 (segment (start 135.89 111.76) (end 133.35 111.76) (width 0.25) (layer "F.Cu") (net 4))
 (segment (start 133.35 111.76) (end 146.13 111.76) (width 0.25) (layer "B.Cu") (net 4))
 (segment (start 157.48 111.76) (end 156.934511 111.214511) (width 0.25) (layer "B.Cu") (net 12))
 (segment (start 156.934511 108.039511) (end 156.21 107.315) (width 0.25) (layer "B.Cu") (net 12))
 (segment (start 163.655 110.95) (end 165.415 112.71) (width 0.25) (layer "B.Cu") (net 12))
 (segment (start 160.655 111.76) (end 161.465 110.95) (width 0.25) (layer "B.Cu") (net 12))
 (segment (start 161.465 110.95) (end 162.88 110.95) (width 0.25) (layer "B.Cu") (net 12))
 (segment (start 159.385 111.76) (end 157.48 111.76) (width 0.25) (layer "B.Cu") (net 12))
 (segment (start 170.99 112.71) (end 170.99 112.22) (width 0.25) (layer "B.Cu") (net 12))
 (segment (start 165.415 112.71) (end 170.99 112.71) (width 0.25) (layer "B.Cu") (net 12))
 (segment (start 162.88 110.95) (end 163.655 110.95) (width 0.25) (layer "B.Cu") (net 12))
 (segment (start 174.07 107.95) (end 174.07 109.855) (width 0.25) (layer "B.Cu") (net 12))
 (segment (start 170.99 112.22) (end 172.085 111.125) (width 0.25) (layer "B.Cu") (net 12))
 (segment (start 172.085 111.125) (end 172.085 109.855) (width 0.25) (layer "B.Cu") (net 12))
 (segment (start 156.934511 111.214511) (end 156.934511 108.039511) (width 0.25) (layer "B.Cu") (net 12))
 (segment (start 174.07 109.855) (end 172.085 109.855) (width 0.25) (layer "B.Cu") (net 12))
 (segment (start 159.385 111.76) (end 160.655 111.76) (width 0.25) (layer "B.Cu") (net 12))
 (segment (start 172.085 107.95) (end 172.085 109.855) (width 0.25) (layer "B.Cu") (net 12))
 (segment (start 159.385 113.19) (end 151.765 113.19) (width 0.25) (layer "F.Cu") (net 2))
 (segment (start 158.053286 111.0355) (end 159.385 112.367214) (width 0.25) (layer "F.Cu") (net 2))
 (segment (start 159.385 112.367214) (end 159.385 113.19) (width 0.25) (layer "F.Cu") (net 2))
 (segment (start 162.56 113.825) (end 161.925 113.19) (width 0.25) (layer "F.Cu") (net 2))
 (segment (start 161.925 113.19) (end 159.385 113.19) (width 0.25) (layer "F.Cu") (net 2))
 (via (at 162.56 113.825) (size 0.8) (drill 0.4) (layers "F.Cu" "B.Cu") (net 2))
 (via (at 158.053286 111.0355) (size 0.8) (drill 0.4) (layers "F.Cu" "B.Cu") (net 2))
 (segment (start 158.053286 111.0355) (end 158.598786 110.49) (width 0.25) (layer "B.Cu") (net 2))
 (segment (start 160.655 110.49) (end 161.93 109.215) (width 0.25) (layer "B.Cu") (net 2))
 (segment (start 161.93 109.215) (end 161.93 107.95) (width 0.25) (layer "B.Cu") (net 2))
 (segment (start 162.6775 113.825) (end 163.4725 113.03) (width 0.25) (layer "B.Cu") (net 2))
 (segment (start 162.56 113.825) (end 162.6775 113.825) (width 0.25) (layer "B.Cu") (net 2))
 (segment (start 159.385 110.49) (end 160.655 110.49) (width 0.25) (layer "B.Cu") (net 2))
 (segment (start 158.598786 110.49) (end 159.385 110.49) (width 0.25) (layer "B.Cu") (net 2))
 (segment (start 168.91 113.438677) (end 168.91 111.710498) (width 0.25) (layer "F.Cu") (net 10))
 (via (at 168.91 111.710498) (size 0.8) (drill 0.4) (layers "F.Cu" "B.Cu") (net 10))
 (via (at 168.91 113.438677) (size 0.8) (drill 0.4) (layers "F.Cu" "B.Cu") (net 10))
 (segment (start 168.0425 108.1025) (end 168.195 107.95) (width 0.25) (layer "B.Cu") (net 10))
 (segment (start 168.0425 109.855) (end 170.01 109.855) (width 0.25) (layer "B.Cu") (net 10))
 (segment (start 168.0425 110.842998) (end 168.0425 109.855) (width 0.25) (layer "B.Cu") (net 10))
 (segment (start 168.91 111.710498) (end 168.0425 110.842998) (width 0.25) (layer "B.Cu") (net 10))
 (segment (start 167.594157 114.75452) (end 150.67202 114.75452) (width 0.25) (layer "B.Cu") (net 10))
 (segment (start 150.67202 114.75452) (end 149.86 113.9425) (width 0.25) (layer "B.Cu") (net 10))
 (segment (start 168.195 107.95) (end 170.26 107.95) (width 0.25) (layer "B.Cu") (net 10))
 (segment (start 168.91 113.438677) (end 167.594157 114.75452) (width 0.25) (layer "B.Cu") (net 10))
 (segment (start 168.0425 109.855) (end 168.0425 108.1025) (width 0.25) (layer "B.Cu") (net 10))
 (segment (start 160.930498 108.359376) (end 160.930498 110.49) (width 0.25) (layer "F.Cu") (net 7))
 (segment (start 175.1 110.49) (end 159.222507 110.49) (width 0.25) (layer "F.Cu") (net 7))
 (segment (start 176.37 111.76) (end 175.1 110.49) (width 0.25) (layer "F.Cu") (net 7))
 (segment (start 158.507507 109.775) (end 153.115 109.775) (width 0.25) (layer "F.Cu") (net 7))
 (segment (start 180.34 110.49) (end 179.07 111.76) (width 0.25) (layer "F.Cu") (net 7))
 (segment (start 179.07 111.76) (end 176.37 111.76) (width 0.25) (layer "F.Cu") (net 7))
 (segment (start 153.115 109.775) (end 153.035 109.855) (width 0.25) (layer "F.Cu") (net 7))
 (segment (start 159.222507 110.49) (end 158.507507 109.775) (width 0.25) (layer "F.Cu") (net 7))
 (via (at 160.930498 108.359376) (size 0.8) (drill 0.4) (layers "F.Cu" "B.Cu") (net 7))
 (via (at 153.035 109.855) (size 0.8) (drill 0.4) (layers "F.Cu" "B.Cu") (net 7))
 (segment (start 159.239376 108.359376) (end 158.195 107.315) (width 0.25) (layer "B.Cu") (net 7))
 (segment (start 153.035 109.855) (end 151.765 109.855) (width 0.25) (layer "B.Cu") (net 7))
 (segment (start 175.895 109.855) (end 175.895 111.335614) (width 0.25) (layer "B.Cu") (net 7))
 (segment (start 175.895 111.335614) (end 176.319397 111.760011) (width 0.25) (layer "B.Cu") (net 7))
 (segment (start 179.069989 111.760011) (end 180.34 110.49) (width 0.25) (layer "B.Cu") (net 7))
 (segment (start 160.930498 108.359376) (end 159.239376 108.359376) (width 0.25) (layer "B.Cu") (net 7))
 (segment (start 176.319397 111.760011) (end 179.069989 111.760011) (width 0.25) (layer "B.Cu") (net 7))
 (segment (start 153.035 111.76) (end 152.6775 112.1175) (width 0.2) (layer "B.Cu") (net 11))
 (segment (start 160.995717 113.03) (end 160.396197 113.62952) (width 0.2) (layer "B.Cu") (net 11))
 (segment (start 161.6475 113.03) (end 160.995717 113.03) (width 0.2) (layer "B.Cu") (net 11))
 (segment (start 155.575 111.76) (end 154.435 111.76) (width 0.2) (layer "B.Cu") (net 11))
 (segment (start 154.435 111.76) (end 153.035 111.76) (width 0.2) (layer "B.Cu") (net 11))
 (segment (start 160.396197 113.62952) (end 157.44452 113.62952) (width 0.2) (layer "B.Cu") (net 11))
 (segment (start 152.6775 112.1175) (end 151.765 112.1175) (width 0.2) (layer "B.Cu") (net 11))
 (segment (start 157.44452 113.62952) (end 155.575 111.76) (width 0.2) (layer "B.Cu") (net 11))
 (segment (start 151.765 107.315) (end 152.56452 106.51548) (width 0.25) (layer "B.Cu") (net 8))
 (segment (start 152.56452 106.51548) (end 174.46048 106.51548) (width 0.25) (layer "B.Cu") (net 8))
 (segment (start 174.46048 106.51548) (end 175.895 107.95) (width 0.25) (layer "B.Cu") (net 8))
 (segment (start 175.895 107.95) (end 180.34 107.95) (width 0.25) (layer "B.Cu") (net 8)))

